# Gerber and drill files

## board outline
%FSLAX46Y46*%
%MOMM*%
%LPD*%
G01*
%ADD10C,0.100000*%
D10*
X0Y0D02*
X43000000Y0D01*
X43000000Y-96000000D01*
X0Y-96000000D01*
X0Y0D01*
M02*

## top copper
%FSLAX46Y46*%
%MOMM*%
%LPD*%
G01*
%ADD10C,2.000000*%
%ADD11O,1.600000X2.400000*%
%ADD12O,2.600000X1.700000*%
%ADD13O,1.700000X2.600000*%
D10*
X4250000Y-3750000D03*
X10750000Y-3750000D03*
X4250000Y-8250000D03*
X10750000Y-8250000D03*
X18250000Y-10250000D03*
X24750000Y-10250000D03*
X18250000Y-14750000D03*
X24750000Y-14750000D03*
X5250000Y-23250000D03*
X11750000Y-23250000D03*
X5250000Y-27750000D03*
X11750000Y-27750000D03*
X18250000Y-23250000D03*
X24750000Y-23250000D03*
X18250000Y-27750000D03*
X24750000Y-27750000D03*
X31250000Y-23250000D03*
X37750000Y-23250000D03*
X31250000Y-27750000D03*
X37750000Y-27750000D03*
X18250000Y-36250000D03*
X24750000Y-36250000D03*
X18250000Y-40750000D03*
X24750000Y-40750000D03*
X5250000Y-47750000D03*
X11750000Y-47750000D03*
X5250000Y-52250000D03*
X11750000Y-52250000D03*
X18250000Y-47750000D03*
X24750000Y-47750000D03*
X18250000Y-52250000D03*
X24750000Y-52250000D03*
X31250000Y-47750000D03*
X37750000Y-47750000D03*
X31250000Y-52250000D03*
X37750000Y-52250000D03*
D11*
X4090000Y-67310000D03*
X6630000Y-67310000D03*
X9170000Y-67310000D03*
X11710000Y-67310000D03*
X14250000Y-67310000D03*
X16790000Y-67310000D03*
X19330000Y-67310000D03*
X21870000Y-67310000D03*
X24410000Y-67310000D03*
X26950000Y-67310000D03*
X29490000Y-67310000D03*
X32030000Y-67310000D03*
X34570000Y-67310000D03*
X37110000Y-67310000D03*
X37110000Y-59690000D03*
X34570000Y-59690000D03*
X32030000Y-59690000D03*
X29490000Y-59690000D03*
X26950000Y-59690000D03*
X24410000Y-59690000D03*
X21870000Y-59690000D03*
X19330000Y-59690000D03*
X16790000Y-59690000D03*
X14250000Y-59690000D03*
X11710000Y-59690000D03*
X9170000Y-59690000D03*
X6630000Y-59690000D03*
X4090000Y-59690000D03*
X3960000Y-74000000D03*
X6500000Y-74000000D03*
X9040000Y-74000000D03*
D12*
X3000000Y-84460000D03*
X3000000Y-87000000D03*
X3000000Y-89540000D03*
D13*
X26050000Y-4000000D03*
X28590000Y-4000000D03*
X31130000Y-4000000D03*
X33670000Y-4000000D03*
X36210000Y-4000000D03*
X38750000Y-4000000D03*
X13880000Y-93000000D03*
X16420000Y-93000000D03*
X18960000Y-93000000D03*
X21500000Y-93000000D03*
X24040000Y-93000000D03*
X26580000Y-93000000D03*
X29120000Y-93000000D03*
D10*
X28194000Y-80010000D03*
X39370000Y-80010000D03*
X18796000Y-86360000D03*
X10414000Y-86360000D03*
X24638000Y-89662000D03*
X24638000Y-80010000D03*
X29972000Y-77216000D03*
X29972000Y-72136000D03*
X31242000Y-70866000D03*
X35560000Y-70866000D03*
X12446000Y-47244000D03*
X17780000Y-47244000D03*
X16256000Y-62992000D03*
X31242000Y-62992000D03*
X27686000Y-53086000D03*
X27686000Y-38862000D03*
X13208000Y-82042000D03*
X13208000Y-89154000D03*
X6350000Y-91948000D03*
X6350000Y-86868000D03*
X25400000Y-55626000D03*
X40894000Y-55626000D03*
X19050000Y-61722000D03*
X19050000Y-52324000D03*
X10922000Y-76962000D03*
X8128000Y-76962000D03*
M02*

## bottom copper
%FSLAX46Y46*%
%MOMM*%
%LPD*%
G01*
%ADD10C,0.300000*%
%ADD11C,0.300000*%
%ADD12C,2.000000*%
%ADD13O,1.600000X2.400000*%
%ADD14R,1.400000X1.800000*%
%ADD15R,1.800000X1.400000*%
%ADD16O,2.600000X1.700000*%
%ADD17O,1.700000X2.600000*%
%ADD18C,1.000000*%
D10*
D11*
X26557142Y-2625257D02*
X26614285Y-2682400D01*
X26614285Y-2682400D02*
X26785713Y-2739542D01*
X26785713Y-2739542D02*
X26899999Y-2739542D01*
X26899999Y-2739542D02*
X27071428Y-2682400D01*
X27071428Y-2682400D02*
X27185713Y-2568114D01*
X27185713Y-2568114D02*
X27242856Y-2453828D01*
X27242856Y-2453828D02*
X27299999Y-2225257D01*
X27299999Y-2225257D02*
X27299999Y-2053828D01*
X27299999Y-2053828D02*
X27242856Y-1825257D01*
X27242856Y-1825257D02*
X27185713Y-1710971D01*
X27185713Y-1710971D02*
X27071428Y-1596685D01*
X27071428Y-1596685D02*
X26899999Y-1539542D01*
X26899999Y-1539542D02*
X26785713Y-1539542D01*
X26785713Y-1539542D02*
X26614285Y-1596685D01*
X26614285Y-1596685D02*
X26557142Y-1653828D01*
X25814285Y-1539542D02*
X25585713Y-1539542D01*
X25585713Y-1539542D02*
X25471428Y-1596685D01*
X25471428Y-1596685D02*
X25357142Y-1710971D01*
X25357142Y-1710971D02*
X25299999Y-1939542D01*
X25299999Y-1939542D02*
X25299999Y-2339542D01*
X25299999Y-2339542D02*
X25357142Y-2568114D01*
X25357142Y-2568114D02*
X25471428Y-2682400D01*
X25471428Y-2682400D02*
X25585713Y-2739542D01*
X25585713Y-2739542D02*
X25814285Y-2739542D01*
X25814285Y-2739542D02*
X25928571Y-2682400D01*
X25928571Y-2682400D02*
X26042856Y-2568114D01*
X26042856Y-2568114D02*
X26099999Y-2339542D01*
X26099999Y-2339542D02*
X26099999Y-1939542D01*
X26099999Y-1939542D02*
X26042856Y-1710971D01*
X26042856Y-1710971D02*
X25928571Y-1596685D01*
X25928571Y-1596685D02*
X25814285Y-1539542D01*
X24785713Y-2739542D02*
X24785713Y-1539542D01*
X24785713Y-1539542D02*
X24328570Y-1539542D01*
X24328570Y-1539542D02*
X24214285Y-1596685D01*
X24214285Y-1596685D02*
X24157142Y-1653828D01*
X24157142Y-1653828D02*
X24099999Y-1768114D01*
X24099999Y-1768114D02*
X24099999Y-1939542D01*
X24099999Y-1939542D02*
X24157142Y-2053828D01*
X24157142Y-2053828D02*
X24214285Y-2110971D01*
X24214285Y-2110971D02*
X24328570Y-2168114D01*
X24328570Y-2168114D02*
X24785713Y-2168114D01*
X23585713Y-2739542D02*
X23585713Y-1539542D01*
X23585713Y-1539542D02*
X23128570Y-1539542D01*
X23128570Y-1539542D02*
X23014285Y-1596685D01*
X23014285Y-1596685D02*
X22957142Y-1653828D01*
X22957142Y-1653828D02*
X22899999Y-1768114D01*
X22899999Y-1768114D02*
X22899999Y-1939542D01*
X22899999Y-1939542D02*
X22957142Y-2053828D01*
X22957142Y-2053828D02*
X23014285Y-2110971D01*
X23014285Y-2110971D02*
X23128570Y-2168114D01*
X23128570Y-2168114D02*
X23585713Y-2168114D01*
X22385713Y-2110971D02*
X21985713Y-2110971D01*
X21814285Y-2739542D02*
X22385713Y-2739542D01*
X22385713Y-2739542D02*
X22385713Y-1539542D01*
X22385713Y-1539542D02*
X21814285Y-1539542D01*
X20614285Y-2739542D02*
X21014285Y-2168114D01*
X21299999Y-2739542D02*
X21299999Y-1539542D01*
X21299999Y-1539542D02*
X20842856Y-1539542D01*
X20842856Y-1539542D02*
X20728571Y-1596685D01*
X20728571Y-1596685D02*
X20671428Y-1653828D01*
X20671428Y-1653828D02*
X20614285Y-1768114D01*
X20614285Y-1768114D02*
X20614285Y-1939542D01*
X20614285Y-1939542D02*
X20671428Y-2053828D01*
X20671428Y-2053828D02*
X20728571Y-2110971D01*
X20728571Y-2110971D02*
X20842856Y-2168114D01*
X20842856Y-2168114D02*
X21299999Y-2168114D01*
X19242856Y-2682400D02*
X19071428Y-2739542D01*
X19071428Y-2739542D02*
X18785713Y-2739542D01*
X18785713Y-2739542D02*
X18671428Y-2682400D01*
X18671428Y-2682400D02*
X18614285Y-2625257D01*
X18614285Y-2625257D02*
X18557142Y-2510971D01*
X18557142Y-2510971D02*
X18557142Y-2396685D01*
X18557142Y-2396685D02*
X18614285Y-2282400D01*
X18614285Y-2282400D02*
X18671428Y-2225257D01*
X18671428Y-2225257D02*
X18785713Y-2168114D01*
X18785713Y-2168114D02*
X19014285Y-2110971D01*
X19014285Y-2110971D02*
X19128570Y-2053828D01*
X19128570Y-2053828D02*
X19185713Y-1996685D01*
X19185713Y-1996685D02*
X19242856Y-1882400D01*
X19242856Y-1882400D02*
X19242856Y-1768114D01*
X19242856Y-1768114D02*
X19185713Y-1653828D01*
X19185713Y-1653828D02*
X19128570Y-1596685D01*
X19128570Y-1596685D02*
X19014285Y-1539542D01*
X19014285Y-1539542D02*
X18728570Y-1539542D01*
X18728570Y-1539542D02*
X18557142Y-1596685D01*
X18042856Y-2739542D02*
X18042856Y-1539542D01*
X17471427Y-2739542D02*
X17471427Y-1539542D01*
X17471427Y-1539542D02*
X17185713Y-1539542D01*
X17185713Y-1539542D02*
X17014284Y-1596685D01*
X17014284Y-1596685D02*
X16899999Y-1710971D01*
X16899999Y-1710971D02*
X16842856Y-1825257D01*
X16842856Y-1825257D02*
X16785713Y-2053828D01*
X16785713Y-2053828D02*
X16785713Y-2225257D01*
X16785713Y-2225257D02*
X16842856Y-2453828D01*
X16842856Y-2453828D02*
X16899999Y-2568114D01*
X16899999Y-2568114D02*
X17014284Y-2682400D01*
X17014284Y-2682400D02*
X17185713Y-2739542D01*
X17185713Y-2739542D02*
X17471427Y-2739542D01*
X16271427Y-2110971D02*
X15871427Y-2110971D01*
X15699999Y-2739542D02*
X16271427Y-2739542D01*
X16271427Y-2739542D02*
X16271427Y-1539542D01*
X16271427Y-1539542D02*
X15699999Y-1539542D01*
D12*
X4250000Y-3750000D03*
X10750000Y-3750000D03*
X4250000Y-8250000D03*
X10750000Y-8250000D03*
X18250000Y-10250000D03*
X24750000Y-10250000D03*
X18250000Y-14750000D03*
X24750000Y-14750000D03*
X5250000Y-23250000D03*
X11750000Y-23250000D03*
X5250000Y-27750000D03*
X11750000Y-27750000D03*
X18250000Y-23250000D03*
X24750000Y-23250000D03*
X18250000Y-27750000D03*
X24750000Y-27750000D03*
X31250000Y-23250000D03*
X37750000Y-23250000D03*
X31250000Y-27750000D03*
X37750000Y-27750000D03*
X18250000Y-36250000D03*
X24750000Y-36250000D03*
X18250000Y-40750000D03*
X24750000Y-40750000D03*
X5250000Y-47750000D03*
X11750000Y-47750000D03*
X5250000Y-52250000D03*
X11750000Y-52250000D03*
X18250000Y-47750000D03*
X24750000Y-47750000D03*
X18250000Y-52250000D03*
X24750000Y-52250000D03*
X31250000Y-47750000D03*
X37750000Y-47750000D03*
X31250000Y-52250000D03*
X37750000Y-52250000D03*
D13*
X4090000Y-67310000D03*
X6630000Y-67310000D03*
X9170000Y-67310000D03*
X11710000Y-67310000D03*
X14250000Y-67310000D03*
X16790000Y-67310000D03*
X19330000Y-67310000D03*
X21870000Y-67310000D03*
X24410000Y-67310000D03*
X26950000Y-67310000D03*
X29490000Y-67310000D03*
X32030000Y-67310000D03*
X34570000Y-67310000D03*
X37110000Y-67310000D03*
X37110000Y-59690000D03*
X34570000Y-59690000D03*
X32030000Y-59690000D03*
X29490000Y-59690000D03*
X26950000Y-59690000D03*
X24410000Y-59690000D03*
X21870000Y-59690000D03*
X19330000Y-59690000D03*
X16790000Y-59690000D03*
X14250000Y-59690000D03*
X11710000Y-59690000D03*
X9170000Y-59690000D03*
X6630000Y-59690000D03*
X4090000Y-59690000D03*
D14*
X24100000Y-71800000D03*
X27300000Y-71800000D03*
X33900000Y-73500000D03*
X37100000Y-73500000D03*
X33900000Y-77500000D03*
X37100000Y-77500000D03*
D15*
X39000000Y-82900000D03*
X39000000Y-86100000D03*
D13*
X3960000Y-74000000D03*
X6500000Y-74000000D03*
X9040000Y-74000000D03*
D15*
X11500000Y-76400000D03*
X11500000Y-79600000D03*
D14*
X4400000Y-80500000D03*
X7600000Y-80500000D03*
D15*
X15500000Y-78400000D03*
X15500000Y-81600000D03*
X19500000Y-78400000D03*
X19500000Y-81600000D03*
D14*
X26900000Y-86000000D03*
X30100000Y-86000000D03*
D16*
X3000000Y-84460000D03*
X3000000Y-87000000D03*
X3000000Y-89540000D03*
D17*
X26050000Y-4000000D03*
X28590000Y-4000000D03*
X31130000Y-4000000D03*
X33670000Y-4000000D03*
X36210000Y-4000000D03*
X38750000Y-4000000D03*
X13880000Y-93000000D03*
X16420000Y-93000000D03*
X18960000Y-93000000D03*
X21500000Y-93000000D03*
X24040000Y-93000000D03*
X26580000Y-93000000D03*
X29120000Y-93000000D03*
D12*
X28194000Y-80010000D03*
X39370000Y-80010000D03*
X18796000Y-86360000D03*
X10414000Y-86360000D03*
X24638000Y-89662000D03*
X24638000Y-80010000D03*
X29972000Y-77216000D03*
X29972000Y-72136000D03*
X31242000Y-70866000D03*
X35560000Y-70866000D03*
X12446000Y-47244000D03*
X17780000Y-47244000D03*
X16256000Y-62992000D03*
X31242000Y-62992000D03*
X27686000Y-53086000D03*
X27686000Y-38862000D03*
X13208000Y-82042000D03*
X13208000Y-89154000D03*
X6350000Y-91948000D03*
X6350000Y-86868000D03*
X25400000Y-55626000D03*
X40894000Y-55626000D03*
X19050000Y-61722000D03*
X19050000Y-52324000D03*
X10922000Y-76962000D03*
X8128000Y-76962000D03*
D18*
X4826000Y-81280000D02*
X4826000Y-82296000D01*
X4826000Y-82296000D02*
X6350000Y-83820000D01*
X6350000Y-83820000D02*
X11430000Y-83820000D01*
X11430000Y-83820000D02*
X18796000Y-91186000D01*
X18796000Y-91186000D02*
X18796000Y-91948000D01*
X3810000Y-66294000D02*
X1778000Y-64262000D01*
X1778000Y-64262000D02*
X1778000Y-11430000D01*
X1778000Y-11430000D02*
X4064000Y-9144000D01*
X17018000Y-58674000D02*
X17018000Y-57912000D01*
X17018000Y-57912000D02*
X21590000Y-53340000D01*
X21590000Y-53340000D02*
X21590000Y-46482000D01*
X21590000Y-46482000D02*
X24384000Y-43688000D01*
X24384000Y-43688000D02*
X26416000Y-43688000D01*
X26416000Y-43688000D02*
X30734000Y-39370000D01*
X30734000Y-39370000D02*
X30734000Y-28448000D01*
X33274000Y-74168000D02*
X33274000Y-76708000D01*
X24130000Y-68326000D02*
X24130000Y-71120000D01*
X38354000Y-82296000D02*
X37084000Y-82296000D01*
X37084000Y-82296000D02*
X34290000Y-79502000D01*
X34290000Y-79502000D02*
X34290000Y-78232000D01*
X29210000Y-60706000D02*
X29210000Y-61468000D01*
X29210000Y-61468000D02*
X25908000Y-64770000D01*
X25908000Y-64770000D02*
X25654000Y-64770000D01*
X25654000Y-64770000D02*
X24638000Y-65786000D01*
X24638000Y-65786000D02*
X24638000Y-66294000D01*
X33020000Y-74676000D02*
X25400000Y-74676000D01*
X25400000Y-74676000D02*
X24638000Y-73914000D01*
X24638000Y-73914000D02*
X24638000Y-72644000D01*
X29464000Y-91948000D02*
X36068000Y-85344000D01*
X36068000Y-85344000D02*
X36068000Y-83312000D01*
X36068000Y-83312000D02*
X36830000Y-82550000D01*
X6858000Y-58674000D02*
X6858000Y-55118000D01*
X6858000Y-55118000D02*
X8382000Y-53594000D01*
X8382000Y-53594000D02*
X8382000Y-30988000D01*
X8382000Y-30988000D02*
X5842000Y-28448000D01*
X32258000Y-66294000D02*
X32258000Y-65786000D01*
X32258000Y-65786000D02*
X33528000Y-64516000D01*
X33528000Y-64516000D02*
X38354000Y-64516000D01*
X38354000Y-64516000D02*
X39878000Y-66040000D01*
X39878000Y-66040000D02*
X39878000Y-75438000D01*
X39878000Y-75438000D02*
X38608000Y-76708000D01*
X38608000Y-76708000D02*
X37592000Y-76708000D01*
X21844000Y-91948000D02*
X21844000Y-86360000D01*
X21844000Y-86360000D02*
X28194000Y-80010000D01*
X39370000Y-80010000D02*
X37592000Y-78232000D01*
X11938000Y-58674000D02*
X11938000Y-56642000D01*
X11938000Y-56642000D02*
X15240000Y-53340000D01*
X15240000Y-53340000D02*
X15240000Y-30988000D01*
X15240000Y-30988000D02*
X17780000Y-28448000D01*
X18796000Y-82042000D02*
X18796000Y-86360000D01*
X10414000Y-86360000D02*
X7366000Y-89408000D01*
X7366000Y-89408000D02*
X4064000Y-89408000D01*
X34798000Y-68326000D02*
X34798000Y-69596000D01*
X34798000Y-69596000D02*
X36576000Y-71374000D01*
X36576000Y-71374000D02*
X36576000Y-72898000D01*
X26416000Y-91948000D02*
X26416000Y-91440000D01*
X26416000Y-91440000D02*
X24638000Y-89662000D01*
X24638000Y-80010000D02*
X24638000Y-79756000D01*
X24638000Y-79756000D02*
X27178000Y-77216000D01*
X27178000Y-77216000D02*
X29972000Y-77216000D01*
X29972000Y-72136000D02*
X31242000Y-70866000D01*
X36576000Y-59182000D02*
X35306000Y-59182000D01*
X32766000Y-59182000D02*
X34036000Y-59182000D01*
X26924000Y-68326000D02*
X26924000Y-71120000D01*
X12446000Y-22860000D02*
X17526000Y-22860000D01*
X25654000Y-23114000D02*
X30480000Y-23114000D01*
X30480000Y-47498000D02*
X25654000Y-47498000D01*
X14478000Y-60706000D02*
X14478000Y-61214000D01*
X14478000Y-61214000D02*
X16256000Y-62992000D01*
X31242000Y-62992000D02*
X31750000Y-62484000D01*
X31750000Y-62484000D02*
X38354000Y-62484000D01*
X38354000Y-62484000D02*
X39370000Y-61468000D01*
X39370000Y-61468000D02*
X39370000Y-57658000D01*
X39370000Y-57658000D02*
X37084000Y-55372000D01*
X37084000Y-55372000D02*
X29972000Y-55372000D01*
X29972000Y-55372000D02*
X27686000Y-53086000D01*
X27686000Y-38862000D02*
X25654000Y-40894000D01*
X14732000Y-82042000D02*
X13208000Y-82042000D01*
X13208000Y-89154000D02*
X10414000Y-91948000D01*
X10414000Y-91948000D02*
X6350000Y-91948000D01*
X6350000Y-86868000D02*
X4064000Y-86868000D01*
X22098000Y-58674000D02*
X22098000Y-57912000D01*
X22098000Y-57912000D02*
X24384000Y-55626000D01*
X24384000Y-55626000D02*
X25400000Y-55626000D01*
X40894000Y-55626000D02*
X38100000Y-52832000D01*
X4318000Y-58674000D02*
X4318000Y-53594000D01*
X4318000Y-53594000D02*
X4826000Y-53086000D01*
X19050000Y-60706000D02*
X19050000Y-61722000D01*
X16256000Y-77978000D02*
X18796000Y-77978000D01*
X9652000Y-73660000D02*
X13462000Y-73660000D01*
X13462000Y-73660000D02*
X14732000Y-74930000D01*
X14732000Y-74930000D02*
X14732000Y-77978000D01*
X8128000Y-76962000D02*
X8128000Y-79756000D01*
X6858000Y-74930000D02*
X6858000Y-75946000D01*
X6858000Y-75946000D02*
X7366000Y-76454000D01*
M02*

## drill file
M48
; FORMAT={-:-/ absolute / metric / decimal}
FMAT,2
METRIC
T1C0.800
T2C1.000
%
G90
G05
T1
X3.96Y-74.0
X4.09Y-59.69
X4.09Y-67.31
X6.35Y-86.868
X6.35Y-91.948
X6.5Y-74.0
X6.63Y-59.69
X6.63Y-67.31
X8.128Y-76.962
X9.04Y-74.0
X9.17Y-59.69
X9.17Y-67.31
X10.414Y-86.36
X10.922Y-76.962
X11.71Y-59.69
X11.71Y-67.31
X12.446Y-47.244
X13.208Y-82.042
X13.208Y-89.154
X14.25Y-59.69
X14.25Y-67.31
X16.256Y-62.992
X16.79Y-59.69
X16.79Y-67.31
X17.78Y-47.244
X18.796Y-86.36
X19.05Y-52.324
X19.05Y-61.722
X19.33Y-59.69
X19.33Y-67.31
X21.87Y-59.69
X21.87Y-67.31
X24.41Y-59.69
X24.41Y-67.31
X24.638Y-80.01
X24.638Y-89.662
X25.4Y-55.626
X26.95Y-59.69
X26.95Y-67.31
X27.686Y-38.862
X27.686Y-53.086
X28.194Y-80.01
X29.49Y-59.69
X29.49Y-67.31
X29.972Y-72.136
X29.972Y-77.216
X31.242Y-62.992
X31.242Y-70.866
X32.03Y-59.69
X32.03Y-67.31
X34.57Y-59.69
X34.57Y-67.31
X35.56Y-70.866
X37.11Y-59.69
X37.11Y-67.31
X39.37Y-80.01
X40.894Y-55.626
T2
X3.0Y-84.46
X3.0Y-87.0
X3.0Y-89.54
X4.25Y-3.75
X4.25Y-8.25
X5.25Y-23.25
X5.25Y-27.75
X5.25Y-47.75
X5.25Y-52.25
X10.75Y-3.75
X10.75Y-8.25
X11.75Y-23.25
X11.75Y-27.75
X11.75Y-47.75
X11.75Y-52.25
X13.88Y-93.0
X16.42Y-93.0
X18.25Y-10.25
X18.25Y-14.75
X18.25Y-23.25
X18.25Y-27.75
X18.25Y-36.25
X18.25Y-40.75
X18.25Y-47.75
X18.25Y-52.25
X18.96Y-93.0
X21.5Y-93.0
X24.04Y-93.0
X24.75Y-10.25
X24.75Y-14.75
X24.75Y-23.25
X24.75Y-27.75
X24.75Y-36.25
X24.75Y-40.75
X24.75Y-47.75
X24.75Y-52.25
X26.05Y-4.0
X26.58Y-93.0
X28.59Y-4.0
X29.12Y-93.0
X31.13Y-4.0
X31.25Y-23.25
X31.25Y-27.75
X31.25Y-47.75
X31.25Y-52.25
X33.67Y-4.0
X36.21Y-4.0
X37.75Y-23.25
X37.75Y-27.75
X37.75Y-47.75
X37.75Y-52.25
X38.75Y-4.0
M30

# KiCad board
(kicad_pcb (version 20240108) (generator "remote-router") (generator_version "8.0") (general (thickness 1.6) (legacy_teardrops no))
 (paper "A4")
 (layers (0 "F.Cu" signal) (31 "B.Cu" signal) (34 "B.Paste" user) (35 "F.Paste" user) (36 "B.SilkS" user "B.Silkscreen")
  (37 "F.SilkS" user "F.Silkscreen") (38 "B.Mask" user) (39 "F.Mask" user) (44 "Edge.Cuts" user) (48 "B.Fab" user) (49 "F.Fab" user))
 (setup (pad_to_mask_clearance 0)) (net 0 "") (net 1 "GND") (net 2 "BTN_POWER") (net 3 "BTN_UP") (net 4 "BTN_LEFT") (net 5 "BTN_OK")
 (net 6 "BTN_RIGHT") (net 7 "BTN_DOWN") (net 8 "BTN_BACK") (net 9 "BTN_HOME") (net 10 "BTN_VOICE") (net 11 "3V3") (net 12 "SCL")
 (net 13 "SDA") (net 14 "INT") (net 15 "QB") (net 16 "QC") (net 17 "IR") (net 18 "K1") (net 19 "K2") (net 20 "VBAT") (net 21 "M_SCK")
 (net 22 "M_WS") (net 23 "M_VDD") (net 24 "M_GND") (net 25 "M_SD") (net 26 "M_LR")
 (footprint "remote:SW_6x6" (layer "F.Cu") (at 7.5000 6.0000)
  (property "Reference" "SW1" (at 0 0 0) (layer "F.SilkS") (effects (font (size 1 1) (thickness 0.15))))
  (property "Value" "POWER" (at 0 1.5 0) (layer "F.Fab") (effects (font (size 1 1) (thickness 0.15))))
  (pad "1" thru_hole circle (at -3.25 -2.25) (size 2.0 2.0) (drill 1.0) (layers "*.Cu" "*.Mask") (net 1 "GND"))
  (pad "2" thru_hole circle (at 3.25 -2.25) (size 2.0 2.0) (drill 1.0) (layers "*.Cu" "*.Mask") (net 1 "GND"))
  (pad "3" thru_hole circle (at -3.25 2.25) (size 2.0 2.0) (drill 1.0) (layers "*.Cu" "*.Mask") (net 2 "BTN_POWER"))
  (pad "4" thru_hole circle (at 3.25 2.25) (size 2.0 2.0) (drill 1.0) (layers "*.Cu" "*.Mask") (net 2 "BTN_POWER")))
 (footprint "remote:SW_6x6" (layer "F.Cu") (at 21.5000 12.5000)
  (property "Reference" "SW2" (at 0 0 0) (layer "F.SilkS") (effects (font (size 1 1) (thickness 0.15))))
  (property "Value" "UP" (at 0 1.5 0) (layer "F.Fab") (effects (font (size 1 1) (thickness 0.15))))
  (pad "1" thru_hole circle (at -3.25 -2.25) (size 2.0 2.0) (drill 1.0) (layers "*.Cu" "*.Mask") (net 1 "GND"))
  (pad "2" thru_hole circle (at 3.25 -2.25) (size 2.0 2.0) (drill 1.0) (layers "*.Cu" "*.Mask") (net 1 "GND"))
  (pad "3" thru_hole circle (at -3.25 2.25) (size 2.0 2.0) (drill 1.0) (layers "*.Cu" "*.Mask") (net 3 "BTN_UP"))
  (pad "4" thru_hole circle (at 3.25 2.25) (size 2.0 2.0) (drill 1.0) (layers "*.Cu" "*.Mask") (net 3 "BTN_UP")))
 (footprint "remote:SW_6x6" (layer "F.Cu") (at 8.5000 25.5000)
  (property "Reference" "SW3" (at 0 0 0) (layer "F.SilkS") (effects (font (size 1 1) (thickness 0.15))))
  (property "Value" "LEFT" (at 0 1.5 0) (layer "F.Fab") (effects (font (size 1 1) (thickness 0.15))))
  (pad "1" thru_hole circle (at -3.25 -2.25) (size 2.0 2.0) (drill 1.0) (layers "*.Cu" "*.Mask") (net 1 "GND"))
  (pad "2" thru_hole circle (at 3.25 -2.25) (size 2.0 2.0) (drill 1.0) (layers "*.Cu" "*.Mask") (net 1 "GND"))
  (pad "3" thru_hole circle (at -3.25 2.25) (size 2.0 2.0) (drill 1.0) (layers "*.Cu" "*.Mask") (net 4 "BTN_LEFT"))
  (pad "4" thru_hole circle (at 3.25 2.25) (size 2.0 2.0) (drill 1.0) (layers "*.Cu" "*.Mask") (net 4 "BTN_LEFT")))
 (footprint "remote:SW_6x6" (layer "F.Cu") (at 21.5000 25.5000)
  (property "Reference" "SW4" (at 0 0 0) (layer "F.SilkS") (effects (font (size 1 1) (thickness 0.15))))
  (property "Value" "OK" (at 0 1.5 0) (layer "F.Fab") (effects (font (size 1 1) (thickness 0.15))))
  (pad "1" thru_hole circle (at -3.25 -2.25) (size 2.0 2.0) (drill 1.0) (layers "*.Cu" "*.Mask") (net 1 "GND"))
  (pad "2" thru_hole circle (at 3.25 -2.25) (size 2.0 2.0) (drill 1.0) (layers "*.Cu" "*.Mask") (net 1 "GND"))
  (pad "3" thru_hole circle (at -3.25 2.25) (size 2.0 2.0) (drill 1.0) (layers "*.Cu" "*.Mask") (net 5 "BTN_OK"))
  (pad "4" thru_hole circle (at 3.25 2.25) (size 2.0 2.0) (drill 1.0) (layers "*.Cu" "*.Mask") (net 5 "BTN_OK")))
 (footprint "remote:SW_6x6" (layer "F.Cu") (at 34.5000 25.5000)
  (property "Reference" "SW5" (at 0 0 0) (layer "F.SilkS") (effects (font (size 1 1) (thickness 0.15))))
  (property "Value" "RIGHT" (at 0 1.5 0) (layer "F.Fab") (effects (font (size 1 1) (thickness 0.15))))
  (pad "1" thru_hole circle (at -3.25 -2.25) (size 2.0 2.0) (drill 1.0) (layers "*.Cu" "*.Mask") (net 1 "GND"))
  (pad "2" thru_hole circle (at 3.25 -2.25) (size 2.0 2.0) (drill 1.0) (layers "*.Cu" "*.Mask") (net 1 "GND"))
  (pad "3" thru_hole circle (at -3.25 2.25) (size 2.0 2.0) (drill 1.0) (layers "*.Cu" "*.Mask") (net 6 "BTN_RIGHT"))
  (pad "4" thru_hole circle (at 3.25 2.25) (size 2.0 2.0) (drill 1.0) (layers "*.Cu" "*.Mask") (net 6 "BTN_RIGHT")))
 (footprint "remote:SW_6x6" (layer "F.Cu") (at 21.5000 38.5000)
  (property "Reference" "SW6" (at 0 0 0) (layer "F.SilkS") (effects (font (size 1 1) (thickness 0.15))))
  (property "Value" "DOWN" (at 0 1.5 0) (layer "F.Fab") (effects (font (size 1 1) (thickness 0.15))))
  (pad "1" thru_hole circle (at -3.25 -2.25) (size 2.0 2.0) (drill 1.0) (layers "*.Cu" "*.Mask") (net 1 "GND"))
  (pad "2" thru_hole circle (at 3.25 -2.25) (size 2.0 2.0) (drill 1.0) (layers "*.Cu" "*.Mask") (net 1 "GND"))
  (pad "3" thru_hole circle (at -3.25 2.25) (size 2.0 2.0) (drill 1.0) (layers "*.Cu" "*.Mask") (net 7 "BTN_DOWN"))
  (pad "4" thru_hole circle (at 3.25 2.25) (size 2.0 2.0) (drill 1.0) (layers "*.Cu" "*.Mask") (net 7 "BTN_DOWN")))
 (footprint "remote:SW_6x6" (layer "F.Cu") (at 8.5000 50.0000)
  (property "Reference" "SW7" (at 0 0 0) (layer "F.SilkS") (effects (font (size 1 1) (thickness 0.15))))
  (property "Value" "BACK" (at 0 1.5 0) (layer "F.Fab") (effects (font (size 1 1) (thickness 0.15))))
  (pad "1" thru_hole circle (at -3.25 -2.25) (size 2.0 2.0) (drill 1.0) (layers "*.Cu" "*.Mask") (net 1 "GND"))
  (pad "2" thru_hole circle (at 3.25 -2.25) (size 2.0 2.0) (drill 1.0) (layers "*.Cu" "*.Mask") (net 1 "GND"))
  (pad "3" thru_hole circle (at -3.25 2.25) (size 2.0 2.0) (drill 1.0) (layers "*.Cu" "*.Mask") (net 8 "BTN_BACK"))
  (pad "4" thru_hole circle (at 3.25 2.25) (size 2.0 2.0) (drill 1.0) (layers "*.Cu" "*.Mask") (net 8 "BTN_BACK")))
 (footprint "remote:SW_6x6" (layer "F.Cu") (at 21.5000 50.0000)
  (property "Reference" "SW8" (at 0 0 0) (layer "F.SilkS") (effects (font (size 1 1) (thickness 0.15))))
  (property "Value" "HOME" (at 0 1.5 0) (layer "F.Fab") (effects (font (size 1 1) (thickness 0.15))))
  (pad "1" thru_hole circle (at -3.25 -2.25) (size 2.0 2.0) (drill 1.0) (layers "*.Cu" "*.Mask") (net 1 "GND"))
  (pad "2" thru_hole circle (at 3.25 -2.25) (size 2.0 2.0) (drill 1.0) (layers "*.Cu" "*.Mask") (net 1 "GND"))
  (pad "3" thru_hole circle (at -3.25 2.25) (size 2.0 2.0) (drill 1.0) (layers "*.Cu" "*.Mask") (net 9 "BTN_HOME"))
  (pad "4" thru_hole circle (at 3.25 2.25) (size 2.0 2.0) (drill 1.0) (layers "*.Cu" "*.Mask") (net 9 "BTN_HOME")))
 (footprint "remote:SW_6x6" (layer "F.Cu") (at 34.5000 50.0000)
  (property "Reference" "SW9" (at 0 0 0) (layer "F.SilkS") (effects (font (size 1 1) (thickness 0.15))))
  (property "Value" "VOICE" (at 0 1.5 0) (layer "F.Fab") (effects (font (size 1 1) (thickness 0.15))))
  (pad "1" thru_hole circle (at -3.25 -2.25) (size 2.0 2.0) (drill 1.0) (layers "*.Cu" "*.Mask") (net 1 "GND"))
  (pad "2" thru_hole circle (at 3.25 -2.25) (size 2.0 2.0) (drill 1.0) (layers "*.Cu" "*.Mask") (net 1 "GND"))
  (pad "3" thru_hole circle (at -3.25 2.25) (size 2.0 2.0) (drill 1.0) (layers "*.Cu" "*.Mask") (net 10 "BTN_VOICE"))
  (pad "4" thru_hole circle (at 3.25 2.25) (size 2.0 2.0) (drill 1.0) (layers "*.Cu" "*.Mask") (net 10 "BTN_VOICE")))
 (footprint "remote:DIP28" (layer "F.Cu") (at 20.6000 63.5000)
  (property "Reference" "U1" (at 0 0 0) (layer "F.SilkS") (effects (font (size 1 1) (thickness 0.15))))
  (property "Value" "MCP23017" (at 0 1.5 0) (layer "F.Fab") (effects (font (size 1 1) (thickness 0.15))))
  (pad "1" thru_hole oval (at -16.51 3.81) (size 1.6 2.4) (drill 0.8) (layers "*.Cu" "*.Mask") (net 2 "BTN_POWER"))
  (pad "2" thru_hole oval (at -13.97 3.81) (size 1.6 2.4) (drill 0.8) (layers "*.Cu" "*.Mask"))
  (pad "3" thru_hole oval (at -11.43 3.81) (size 1.6 2.4) (drill 0.8) (layers "*.Cu" "*.Mask"))
  (pad "4" thru_hole oval (at -8.89 3.81) (size 1.6 2.4) (drill 0.8) (layers "*.Cu" "*.Mask"))
  (pad "5" thru_hole oval (at -6.35 3.81) (size 1.6 2.4) (drill 0.8) (layers "*.Cu" "*.Mask"))
  (pad "6" thru_hole oval (at -3.81 3.81) (size 1.6 2.4) (drill 0.8) (layers "*.Cu" "*.Mask"))
  (pad "7" thru_hole oval (at -1.27 3.81) (size 1.6 2.4) (drill 0.8) (layers "*.Cu" "*.Mask"))
  (pad "8" thru_hole oval (at 1.27 3.81) (size 1.6 2.4) (drill 0.8) (layers "*.Cu" "*.Mask"))
  (pad "9" thru_hole oval (at 3.81 3.81) (size 1.6 2.4) (drill 0.8) (layers "*.Cu" "*.Mask") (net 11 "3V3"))
  (pad "10" thru_hole oval (at 6.35 3.81) (size 1.6 2.4) (drill 0.8) (layers "*.Cu" "*.Mask") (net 1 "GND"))
  (pad "11" thru_hole oval (at 8.89 3.81) (size 1.6 2.4) (drill 0.8) (layers "*.Cu" "*.Mask"))
  (pad "12" thru_hole oval (at 11.43 3.81) (size 1.6 2.4) (drill 0.8) (layers "*.Cu" "*.Mask") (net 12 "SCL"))
  (pad "13" thru_hole oval (at 13.97 3.81) (size 1.6 2.4) (drill 0.8) (layers "*.Cu" "*.Mask") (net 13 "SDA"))
  (pad "14" thru_hole oval (at 16.51 3.81) (size 1.6 2.4) (drill 0.8) (layers "*.Cu" "*.Mask"))
  (pad "15" thru_hole oval (at 16.51 -3.81) (size 1.6 2.4) (drill 0.8) (layers "*.Cu" "*.Mask") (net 1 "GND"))
  (pad "16" thru_hole oval (at 13.97 -3.81) (size 1.6 2.4) (drill 0.8) (layers "*.Cu" "*.Mask") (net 1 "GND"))
  (pad "17" thru_hole oval (at 11.43 -3.81) (size 1.6 2.4) (drill 0.8) (layers "*.Cu" "*.Mask") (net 1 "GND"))
  (pad "18" thru_hole oval (at 8.89 -3.81) (size 1.6 2.4) (drill 0.8) (layers "*.Cu" "*.Mask") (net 11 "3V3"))
  (pad "19" thru_hole oval (at 6.35 -3.81) (size 1.6 2.4) (drill 0.8) (layers "*.Cu" "*.Mask"))
  (pad "20" thru_hole oval (at 3.81 -3.81) (size 1.6 2.4) (drill 0.8) (layers "*.Cu" "*.Mask") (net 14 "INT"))
  (pad "21" thru_hole oval (at 1.27 -3.81) (size 1.6 2.4) (drill 0.8) (layers "*.Cu" "*.Mask") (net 10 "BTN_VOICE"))
  (pad "22" thru_hole oval (at -1.27 -3.81) (size 1.6 2.4) (drill 0.8) (layers "*.Cu" "*.Mask") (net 9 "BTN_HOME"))
  (pad "23" thru_hole oval (at -3.81 -3.81) (size 1.6 2.4) (drill 0.8) (layers "*.Cu" "*.Mask") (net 6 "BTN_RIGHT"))
  (pad "24" thru_hole oval (at -6.35 -3.81) (size 1.6 2.4) (drill 0.8) (layers "*.Cu" "*.Mask") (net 7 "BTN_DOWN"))
  (pad "25" thru_hole oval (at -8.89 -3.81) (size 1.6 2.4) (drill 0.8) (layers "*.Cu" "*.Mask") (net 5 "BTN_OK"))
  (pad "26" thru_hole oval (at -11.43 -3.81) (size 1.6 2.4) (drill 0.8) (layers "*.Cu" "*.Mask") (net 3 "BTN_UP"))
  (pad "27" thru_hole oval (at -13.97 -3.81) (size 1.6 2.4) (drill 0.8) (layers "*.Cu" "*.Mask") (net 4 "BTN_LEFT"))
  (pad "28" thru_hole oval (at -16.51 -3.81) (size 1.6 2.4) (drill 0.8) (layers "*.Cu" "*.Mask") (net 8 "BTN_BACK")))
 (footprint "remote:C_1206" (layer "F.Cu") (at 25.7000 71.8000)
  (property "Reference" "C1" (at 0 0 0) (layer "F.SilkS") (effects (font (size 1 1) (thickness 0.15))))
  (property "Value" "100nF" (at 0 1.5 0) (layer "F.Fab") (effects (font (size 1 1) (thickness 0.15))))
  (pad "1" smd rect (at -1.6 0.0) (size 1.4 1.8) (layers "B.Cu" "B.Mask") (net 11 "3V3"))
  (pad "2" smd rect (at 1.6 0.0) (size 1.4 1.8) (layers "B.Cu" "B.Mask") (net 1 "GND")))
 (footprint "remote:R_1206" (layer "F.Cu") (at 35.5000 73.5000)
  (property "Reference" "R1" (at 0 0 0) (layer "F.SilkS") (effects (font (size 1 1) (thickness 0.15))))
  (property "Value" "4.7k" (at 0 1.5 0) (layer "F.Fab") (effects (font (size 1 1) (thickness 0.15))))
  (pad "1" smd rect (at -1.6 0.0) (size 1.4 1.8) (layers "B.Cu" "B.Mask") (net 11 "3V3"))
  (pad "2" smd rect (at 1.6 0.0) (size 1.4 1.8) (layers "B.Cu" "B.Mask") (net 13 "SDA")))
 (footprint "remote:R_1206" (layer "F.Cu") (at 35.5000 77.5000)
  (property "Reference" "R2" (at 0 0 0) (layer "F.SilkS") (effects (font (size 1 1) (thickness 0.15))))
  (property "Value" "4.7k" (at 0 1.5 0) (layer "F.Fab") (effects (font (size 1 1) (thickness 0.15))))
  (pad "1" smd rect (at -1.6 0.0) (size 1.4 1.8) (layers "B.Cu" "B.Mask") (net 11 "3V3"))
  (pad "2" smd rect (at 1.6 0.0) (size 1.4 1.8) (layers "B.Cu" "B.Mask") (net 12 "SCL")))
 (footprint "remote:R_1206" (layer "F.Cu") (at 39.0000 84.5000)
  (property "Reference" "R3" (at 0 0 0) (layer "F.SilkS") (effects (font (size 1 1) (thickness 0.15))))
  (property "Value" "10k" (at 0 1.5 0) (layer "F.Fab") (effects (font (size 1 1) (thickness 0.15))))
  (pad "1" smd rect (at 0.0 -1.6) (size 1.8 1.4) (layers "B.Cu" "B.Mask") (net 11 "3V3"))
  (pad "2" smd rect (at 0.0 1.6) (size 1.8 1.4) (layers "B.Cu" "B.Mask") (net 14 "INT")))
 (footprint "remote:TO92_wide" (layer "F.Cu") (at 6.5000 74.0000)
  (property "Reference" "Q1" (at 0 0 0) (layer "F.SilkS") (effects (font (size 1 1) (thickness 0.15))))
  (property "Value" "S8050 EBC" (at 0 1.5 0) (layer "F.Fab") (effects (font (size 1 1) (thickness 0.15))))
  (pad "E" thru_hole oval (at -2.54 0.0) (size 1.6 2.4) (drill 0.8) (layers "*.Cu" "*.Mask") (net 1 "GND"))
  (pad "B" thru_hole oval (at 0.0 0.0) (size 1.6 2.4) (drill 0.8) (layers "*.Cu" "*.Mask") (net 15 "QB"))
  (pad "C" thru_hole oval (at 2.54 0.0) (size 1.6 2.4) (drill 0.8) (layers "*.Cu" "*.Mask") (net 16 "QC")))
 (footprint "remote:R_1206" (layer "F.Cu") (at 11.5000 78.0000)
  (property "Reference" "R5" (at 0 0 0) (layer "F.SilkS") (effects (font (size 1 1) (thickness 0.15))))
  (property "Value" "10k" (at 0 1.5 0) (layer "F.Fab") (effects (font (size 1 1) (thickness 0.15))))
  (pad "1" smd rect (at 0.0 -1.6) (size 1.8 1.4) (layers "B.Cu" "B.Mask") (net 15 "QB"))
  (pad "2" smd rect (at 0.0 1.6) (size 1.8 1.4) (layers "B.Cu" "B.Mask") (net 1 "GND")))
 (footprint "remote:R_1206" (layer "F.Cu") (at 6.0000 80.5000)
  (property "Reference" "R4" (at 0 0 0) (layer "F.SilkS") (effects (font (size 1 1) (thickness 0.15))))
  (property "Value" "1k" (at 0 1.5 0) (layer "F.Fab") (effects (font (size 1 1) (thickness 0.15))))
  (pad "1" smd rect (at -1.6 0.0) (size 1.4 1.8) (layers "B.Cu" "B.Mask") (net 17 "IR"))
  (pad "2" smd rect (at 1.6 0.0) (size 1.4 1.8) (layers "B.Cu" "B.Mask") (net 15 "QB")))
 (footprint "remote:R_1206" (layer "F.Cu") (at 15.5000 80.0000)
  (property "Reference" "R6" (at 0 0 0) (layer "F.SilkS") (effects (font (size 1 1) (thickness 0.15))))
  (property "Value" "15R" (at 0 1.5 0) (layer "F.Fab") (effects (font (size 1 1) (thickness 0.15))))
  (pad "1" smd rect (at 0.0 -1.6) (size 1.8 1.4) (layers "B.Cu" "B.Mask") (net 16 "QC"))
  (pad "2" smd rect (at 0.0 1.6) (size 1.8 1.4) (layers "B.Cu" "B.Mask") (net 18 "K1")))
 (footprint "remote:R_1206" (layer "F.Cu") (at 19.5000 80.0000)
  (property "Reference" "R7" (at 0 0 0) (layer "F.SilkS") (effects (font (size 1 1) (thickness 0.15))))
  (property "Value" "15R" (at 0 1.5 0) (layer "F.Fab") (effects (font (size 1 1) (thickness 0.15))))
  (pad "1" smd rect (at 0.0 -1.6) (size 1.8 1.4) (layers "B.Cu" "B.Mask") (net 16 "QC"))
  (pad "2" smd rect (at 0.0 1.6) (size 1.8 1.4) (layers "B.Cu" "B.Mask") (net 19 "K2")))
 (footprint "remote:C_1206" (layer "F.Cu") (at 28.5000 86.0000)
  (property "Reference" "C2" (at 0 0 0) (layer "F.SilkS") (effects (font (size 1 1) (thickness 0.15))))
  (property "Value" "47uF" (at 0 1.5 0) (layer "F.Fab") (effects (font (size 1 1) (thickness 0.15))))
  (pad "1" smd rect (at -1.6 0.0) (size 1.4 1.8) (layers "B.Cu" "B.Mask") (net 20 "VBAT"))
  (pad "2" smd rect (at 1.6 0.0) (size 1.4 1.8) (layers "B.Cu" "B.Mask") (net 1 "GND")))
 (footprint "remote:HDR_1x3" (layer "F.Cu") (at 3.0000 87.0000)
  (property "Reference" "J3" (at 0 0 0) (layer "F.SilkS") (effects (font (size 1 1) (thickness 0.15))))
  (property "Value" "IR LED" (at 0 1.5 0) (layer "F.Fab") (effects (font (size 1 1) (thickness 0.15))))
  (pad "1" thru_hole oval (at 0.0 -2.54) (size 2.6 1.7) (drill 1.0) (layers "*.Cu" "*.Mask") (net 20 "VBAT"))
  (pad "2" thru_hole oval (at 0.0 0.0) (size 2.6 1.7) (drill 1.0) (layers "*.Cu" "*.Mask") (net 18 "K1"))
  (pad "3" thru_hole oval (at 0.0 2.54) (size 2.6 1.7) (drill 1.0) (layers "*.Cu" "*.Mask") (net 19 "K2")))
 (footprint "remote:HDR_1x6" (layer "F.Cu") (at 32.4000 4.0000)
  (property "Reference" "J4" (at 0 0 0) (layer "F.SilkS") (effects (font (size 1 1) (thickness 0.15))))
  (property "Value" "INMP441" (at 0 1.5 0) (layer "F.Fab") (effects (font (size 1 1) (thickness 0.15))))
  (pad "1" thru_hole oval (at -6.35 0.0) (size 1.7 2.6) (drill 1.0) (layers "*.Cu" "*.Mask") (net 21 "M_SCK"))
  (pad "2" thru_hole oval (at -3.81 0.0) (size 1.7 2.6) (drill 1.0) (layers "*.Cu" "*.Mask") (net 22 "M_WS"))
  (pad "3" thru_hole oval (at -1.27 0.0) (size 1.7 2.6) (drill 1.0) (layers "*.Cu" "*.Mask") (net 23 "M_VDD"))
  (pad "4" thru_hole oval (at 1.27 0.0) (size 1.7 2.6) (drill 1.0) (layers "*.Cu" "*.Mask") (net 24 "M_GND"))
  (pad "5" thru_hole oval (at 3.81 0.0) (size 1.7 2.6) (drill 1.0) (layers "*.Cu" "*.Mask") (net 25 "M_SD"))
  (pad "6" thru_hole oval (at 6.35 0.0) (size 1.7 2.6) (drill 1.0) (layers "*.Cu" "*.Mask") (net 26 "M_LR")))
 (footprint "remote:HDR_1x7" (layer "F.Cu") (at 21.5000 93.0000)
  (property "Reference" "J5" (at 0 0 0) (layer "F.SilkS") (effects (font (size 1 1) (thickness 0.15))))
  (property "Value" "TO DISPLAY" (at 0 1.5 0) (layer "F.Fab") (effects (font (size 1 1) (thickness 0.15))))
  (pad "1" thru_hole oval (at -7.62 0.0) (size 1.7 2.6) (drill 1.0) (layers "*.Cu" "*.Mask") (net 20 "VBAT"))
  (pad "2" thru_hole oval (at -5.08 0.0) (size 1.7 2.6) (drill 1.0) (layers "*.Cu" "*.Mask") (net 14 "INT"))
  (pad "3" thru_hole oval (at -2.54 0.0) (size 1.7 2.6) (drill 1.0) (layers "*.Cu" "*.Mask") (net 17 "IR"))
  (pad "4" thru_hole oval (at 0.0 0.0) (size 1.7 2.6) (drill 1.0) (layers "*.Cu" "*.Mask") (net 12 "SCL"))
  (pad "5" thru_hole oval (at 2.54 0.0) (size 1.7 2.6) (drill 1.0) (layers "*.Cu" "*.Mask") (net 1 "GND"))
  (pad "6" thru_hole oval (at 5.08 0.0) (size 1.7 2.6) (drill 1.0) (layers "*.Cu" "*.Mask") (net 13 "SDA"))
  (pad "7" thru_hole oval (at 7.62 0.0) (size 1.7 2.6) (drill 1.0) (layers "*.Cu" "*.Mask") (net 11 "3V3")))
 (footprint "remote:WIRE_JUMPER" (layer "F.Cu") (at 33.7820 80.0100)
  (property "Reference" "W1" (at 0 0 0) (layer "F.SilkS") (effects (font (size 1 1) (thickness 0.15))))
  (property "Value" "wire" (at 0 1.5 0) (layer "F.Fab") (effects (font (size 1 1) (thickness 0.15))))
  (pad "1" thru_hole circle (at -5.588 0.0) (size 2.0 2.0) (drill 0.8) (layers "*.Cu" "*.Mask") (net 12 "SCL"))
  (pad "2" thru_hole circle (at 5.588 0.0) (size 2.0 2.0) (drill 0.8) (layers "*.Cu" "*.Mask") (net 12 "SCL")))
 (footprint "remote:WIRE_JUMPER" (layer "F.Cu") (at 14.6050 86.3600)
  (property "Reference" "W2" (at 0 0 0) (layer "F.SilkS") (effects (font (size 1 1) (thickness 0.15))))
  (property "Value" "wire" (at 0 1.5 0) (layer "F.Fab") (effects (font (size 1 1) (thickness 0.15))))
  (pad "1" thru_hole circle (at 4.191 0.0) (size 2.0 2.0) (drill 0.8) (layers "*.Cu" "*.Mask") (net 19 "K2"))
  (pad "2" thru_hole circle (at -4.191 0.0) (size 2.0 2.0) (drill 0.8) (layers "*.Cu" "*.Mask") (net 19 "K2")))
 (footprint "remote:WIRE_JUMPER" (layer "F.Cu") (at 24.6380 84.8360)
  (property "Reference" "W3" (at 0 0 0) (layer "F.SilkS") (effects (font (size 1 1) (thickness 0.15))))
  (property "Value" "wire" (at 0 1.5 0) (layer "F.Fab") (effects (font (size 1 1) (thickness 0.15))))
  (pad "1" thru_hole circle (at 0.0 4.826) (size 2.0 2.0) (drill 0.8) (layers "*.Cu" "*.Mask") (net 13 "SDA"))
  (pad "2" thru_hole circle (at 0.0 -4.826) (size 2.0 2.0) (drill 0.8) (layers "*.Cu" "*.Mask") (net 13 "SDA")))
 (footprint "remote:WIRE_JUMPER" (layer "F.Cu") (at 29.9720 74.6760)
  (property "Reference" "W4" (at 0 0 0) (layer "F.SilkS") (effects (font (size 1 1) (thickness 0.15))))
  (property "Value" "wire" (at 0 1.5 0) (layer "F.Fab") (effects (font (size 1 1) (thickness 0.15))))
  (pad "1" thru_hole circle (at 0.0 2.54) (size 2.0 2.0) (drill 0.8) (layers "*.Cu" "*.Mask") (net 13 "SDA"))
  (pad "2" thru_hole circle (at 0.0 -2.54) (size 2.0 2.0) (drill 0.8) (layers "*.Cu" "*.Mask") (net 13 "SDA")))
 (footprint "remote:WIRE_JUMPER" (layer "F.Cu") (at 33.4010 70.8660)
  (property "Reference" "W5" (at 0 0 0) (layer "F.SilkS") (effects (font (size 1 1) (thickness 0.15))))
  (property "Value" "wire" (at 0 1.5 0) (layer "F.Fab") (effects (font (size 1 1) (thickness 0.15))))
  (pad "1" thru_hole circle (at -2.159 0.0) (size 2.0 2.0) (drill 0.8) (layers "*.Cu" "*.Mask") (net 13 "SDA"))
  (pad "2" thru_hole circle (at 2.159 0.0) (size 2.0 2.0) (drill 0.8) (layers "*.Cu" "*.Mask") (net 13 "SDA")))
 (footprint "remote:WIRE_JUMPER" (layer "F.Cu") (at 15.1130 47.2440)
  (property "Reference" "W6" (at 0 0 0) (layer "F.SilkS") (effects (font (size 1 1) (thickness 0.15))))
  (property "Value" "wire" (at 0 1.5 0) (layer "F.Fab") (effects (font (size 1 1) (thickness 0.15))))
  (pad "1" thru_hole circle (at -2.667 0.0) (size 2.0 2.0) (drill 0.8) (layers "*.Cu" "*.Mask") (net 1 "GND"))
  (pad "2" thru_hole circle (at 2.667 0.0) (size 2.0 2.0) (drill 0.8) (layers "*.Cu" "*.Mask") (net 1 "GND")))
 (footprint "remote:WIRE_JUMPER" (layer "F.Cu") (at 23.7490 62.9920)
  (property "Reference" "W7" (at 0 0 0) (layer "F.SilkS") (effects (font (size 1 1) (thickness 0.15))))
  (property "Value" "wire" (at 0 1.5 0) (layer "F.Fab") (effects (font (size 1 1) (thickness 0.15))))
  (pad "1" thru_hole circle (at -7.493 0.0) (size 2.0 2.0) (drill 0.8) (layers "*.Cu" "*.Mask") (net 7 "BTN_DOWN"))
  (pad "2" thru_hole circle (at 7.493 0.0) (size 2.0 2.0) (drill 0.8) (layers "*.Cu" "*.Mask") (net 7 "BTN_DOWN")))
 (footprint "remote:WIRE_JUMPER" (layer "F.Cu") (at 27.6860 45.9740)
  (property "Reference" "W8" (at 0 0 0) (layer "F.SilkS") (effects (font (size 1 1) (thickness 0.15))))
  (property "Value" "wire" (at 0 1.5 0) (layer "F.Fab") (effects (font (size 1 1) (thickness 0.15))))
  (pad "1" thru_hole circle (at 0.0 7.112) (size 2.0 2.0) (drill 0.8) (layers "*.Cu" "*.Mask") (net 7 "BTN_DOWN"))
  (pad "2" thru_hole circle (at 0.0 -7.112) (size 2.0 2.0) (drill 0.8) (layers "*.Cu" "*.Mask") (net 7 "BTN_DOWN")))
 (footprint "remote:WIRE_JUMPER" (layer "F.Cu") (at 13.2080 85.5980)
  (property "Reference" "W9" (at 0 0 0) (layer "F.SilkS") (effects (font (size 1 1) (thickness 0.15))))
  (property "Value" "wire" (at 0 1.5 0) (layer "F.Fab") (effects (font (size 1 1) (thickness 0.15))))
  (pad "1" thru_hole circle (at 0.0 -3.556) (size 2.0 2.0) (drill 0.8) (layers "*.Cu" "*.Mask") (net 18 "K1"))
  (pad "2" thru_hole circle (at 0.0 3.556) (size 2.0 2.0) (drill 0.8) (layers "*.Cu" "*.Mask") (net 18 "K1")))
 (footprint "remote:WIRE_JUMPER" (layer "F.Cu") (at 6.3500 89.4080)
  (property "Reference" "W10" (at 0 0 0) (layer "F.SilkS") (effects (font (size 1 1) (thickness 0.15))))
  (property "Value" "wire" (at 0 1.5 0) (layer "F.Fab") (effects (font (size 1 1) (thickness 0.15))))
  (pad "1" thru_hole circle (at 0.0 2.54) (size 2.0 2.0) (drill 0.8) (layers "*.Cu" "*.Mask") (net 18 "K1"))
  (pad "2" thru_hole circle (at 0.0 -2.54) (size 2.0 2.0) (drill 0.8) (layers "*.Cu" "*.Mask") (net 18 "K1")))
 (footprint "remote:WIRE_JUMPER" (layer "F.Cu") (at 33.1470 55.6260)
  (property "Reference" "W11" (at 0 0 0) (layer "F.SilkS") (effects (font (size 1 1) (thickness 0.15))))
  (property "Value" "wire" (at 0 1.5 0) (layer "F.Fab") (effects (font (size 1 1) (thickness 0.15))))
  (pad "1" thru_hole circle (at -7.747 0.0) (size 2.0 2.0) (drill 0.8) (layers "*.Cu" "*.Mask") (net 10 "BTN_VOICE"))
  (pad "2" thru_hole circle (at 7.747 0.0) (size 2.0 2.0) (drill 0.8) (layers "*.Cu" "*.Mask") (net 10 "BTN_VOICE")))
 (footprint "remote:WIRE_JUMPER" (layer "F.Cu") (at 19.0500 57.0230)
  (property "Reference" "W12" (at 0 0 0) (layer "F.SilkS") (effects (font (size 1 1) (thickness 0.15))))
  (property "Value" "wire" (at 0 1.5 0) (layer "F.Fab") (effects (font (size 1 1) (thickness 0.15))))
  (pad "1" thru_hole circle (at 0.0 4.699) (size 2.0 2.0) (drill 0.8) (layers "*.Cu" "*.Mask") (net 9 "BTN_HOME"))
  (pad "2" thru_hole circle (at 0.0 -4.699) (size 2.0 2.0) (drill 0.8) (layers "*.Cu" "*.Mask") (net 9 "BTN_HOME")))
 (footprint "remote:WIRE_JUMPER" (layer "F.Cu") (at 9.5250 76.9620)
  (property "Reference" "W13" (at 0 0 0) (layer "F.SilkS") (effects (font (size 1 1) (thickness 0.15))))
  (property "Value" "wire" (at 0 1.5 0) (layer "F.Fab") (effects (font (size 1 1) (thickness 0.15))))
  (pad "1" thru_hole circle (at 1.397 0.0) (size 2.0 2.0) (drill 0.8) (layers "*.Cu" "*.Mask") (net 15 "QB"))
  (pad "2" thru_hole circle (at -1.397 0.0) (size 2.0 2.0) (drill 0.8) (layers "*.Cu" "*.Mask") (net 15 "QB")))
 (segment (start 4.8260 81.2800) (end 4.8260 82.2960) (width 1.0) (layer "B.Cu") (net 17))
 (segment (start 4.8260 82.2960) (end 6.3500 83.8200) (width 1.0) (layer "B.Cu") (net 17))
 (segment (start 6.3500 83.8200) (end 11.4300 83.8200) (width 1.0) (layer "B.Cu") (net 17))
 (segment (start 11.4300 83.8200) (end 18.7960 91.1860) (width 1.0) (layer "B.Cu") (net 17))
 (segment (start 18.7960 91.1860) (end 18.7960 91.9480) (width 1.0) (layer "B.Cu") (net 17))
 (segment (start 3.8100 66.2940) (end 1.7780 64.2620) (width 1.0) (layer "B.Cu") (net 2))
 (segment (start 1.7780 64.2620) (end 1.7780 11.4300) (width 1.0) (layer "B.Cu") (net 2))
 (segment (start 1.7780 11.4300) (end 4.0640 9.1440) (width 1.0) (layer "B.Cu") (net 2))
 (segment (start 17.0180 58.6740) (end 17.0180 57.9120) (width 1.0) (layer "B.Cu") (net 6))
 (segment (start 17.0180 57.9120) (end 21.5900 53.3400) (width 1.0) (layer "B.Cu") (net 6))
 (segment (start 21.5900 53.3400) (end 21.5900 46.4820) (width 1.0) (layer "B.Cu") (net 6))
 (segment (start 21.5900 46.4820) (end 24.3840 43.6880) (width 1.0) (layer "B.Cu") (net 6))
 (segment (start 24.3840 43.6880) (end 26.4160 43.6880) (width 1.0) (layer "B.Cu") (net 6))
 (segment (start 26.4160 43.6880) (end 30.7340 39.3700) (width 1.0) (layer "B.Cu") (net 6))
 (segment (start 30.7340 39.3700) (end 30.7340 28.4480) (width 1.0) (layer "B.Cu") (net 6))
 (segment (start 33.2740 74.1680) (end 33.2740 76.7080) (width 1.0) (layer "B.Cu") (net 11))
 (segment (start 24.1300 68.3260) (end 24.1300 71.1200) (width 1.0) (layer "B.Cu") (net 11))
 (segment (start 38.3540 82.2960) (end 37.0840 82.2960) (width 1.0) (layer "B.Cu") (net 11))
 (segment (start 37.0840 82.2960) (end 34.2900 79.5020) (width 1.0) (layer "B.Cu") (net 11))
 (segment (start 34.2900 79.5020) (end 34.2900 78.2320) (width 1.0) (layer "B.Cu") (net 11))
 (segment (start 29.2100 60.7060) (end 29.2100 61.4680) (width 1.0) (layer "B.Cu") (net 11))
 (segment (start 29.2100 61.4680) (end 25.9080 64.7700) (width 1.0) (layer "B.Cu") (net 11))
 (segment (start 25.9080 64.7700) (end 25.6540 64.7700) (width 1.0) (layer "B.Cu") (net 11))
 (segment (start 25.6540 64.7700) (end 24.6380 65.7860) (width 1.0) (layer "B.Cu") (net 11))
 (segment (start 24.6380 65.7860) (end 24.6380 66.2940) (width 1.0) (layer "B.Cu") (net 11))
 (segment (start 33.0200 74.6760) (end 25.4000 74.6760) (width 1.0) (layer "B.Cu") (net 11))
 (segment (start 25.4000 74.6760) (end 24.6380 73.9140) (width 1.0) (layer "B.Cu") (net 11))
 (segment (start 24.6380 73.9140) (end 24.6380 72.6440) (width 1.0) (layer "B.Cu") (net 11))
 (segment (start 29.4640 91.9480) (end 36.0680 85.3440) (width 1.0) (layer "B.Cu") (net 11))
 (segment (start 36.0680 85.3440) (end 36.0680 83.3120) (width 1.0) (layer "B.Cu") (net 11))
 (segment (start 36.0680 83.3120) (end 36.8300 82.5500) (width 1.0) (layer "B.Cu") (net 11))
 (segment (start 6.8580 58.6740) (end 6.8580 55.1180) (width 1.0) (layer "B.Cu") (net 4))
 (segment (start 6.8580 55.1180) (end 8.3820 53.5940) (width 1.0) (layer "B.Cu") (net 4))
 (segment (start 8.3820 53.5940) (end 8.3820 30.9880) (width 1.0) (layer "B.Cu") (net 4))
 (segment (start 8.3820 30.9880) (end 5.8420 28.4480) (width 1.0) (layer "B.Cu") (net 4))
 (segment (start 32.2580 66.2940) (end 32.2580 65.7860) (width 1.0) (layer "B.Cu") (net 12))
 (segment (start 32.2580 65.7860) (end 33.5280 64.5160) (width 1.0) (layer "B.Cu") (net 12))
 (segment (start 33.5280 64.5160) (end 38.3540 64.5160) (width 1.0) (layer "B.Cu") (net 12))
 (segment (start 38.3540 64.5160) (end 39.8780 66.0400) (width 1.0) (layer "B.Cu") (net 12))
 (segment (start 39.8780 66.0400) (end 39.8780 75.4380) (width 1.0) (layer "B.Cu") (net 12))
 (segment (start 39.8780 75.4380) (end 38.6080 76.7080) (width 1.0) (layer "B.Cu") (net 12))
 (segment (start 38.6080 76.7080) (end 37.5920 76.7080) (width 1.0) (layer "B.Cu") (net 12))
 (segment (start 21.8440 91.9480) (end 21.8440 86.3600) (width 1.0) (layer "B.Cu") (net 12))
 (segment (start 21.8440 86.3600) (end 28.1940 80.0100) (width 1.0) (layer "B.Cu") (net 12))
 (segment (start 39.3700 80.0100) (end 37.5920 78.2320) (width 1.0) (layer "B.Cu") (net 12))
 (segment (start 11.9380 58.6740) (end 11.9380 56.6420) (width 1.0) (layer "B.Cu") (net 5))
 (segment (start 11.9380 56.6420) (end 15.2400 53.3400) (width 1.0) (layer "B.Cu") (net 5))
 (segment (start 15.2400 53.3400) (end 15.2400 30.9880) (width 1.0) (layer "B.Cu") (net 5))
 (segment (start 15.2400 30.9880) (end 17.7800 28.4480) (width 1.0) (layer "B.Cu") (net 5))
 (segment (start 18.7960 82.0420) (end 18.7960 86.3600) (width 1.0) (layer "B.Cu") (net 19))
 (segment (start 10.4140 86.3600) (end 7.3660 89.4080) (width 1.0) (layer "B.Cu") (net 19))
 (segment (start 7.3660 89.4080) (end 4.0640 89.4080) (width 1.0) (layer "B.Cu") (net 19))
 (segment (start 34.7980 68.3260) (end 34.7980 69.5960) (width 1.0) (layer "B.Cu") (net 13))
 (segment (start 34.7980 69.5960) (end 36.5760 71.3740) (width 1.0) (layer "B.Cu") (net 13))
 (segment (start 36.5760 71.3740) (end 36.5760 72.8980) (width 1.0) (layer "B.Cu") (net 13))
 (segment (start 26.4160 91.9480) (end 26.4160 91.4400) (width 1.0) (layer "B.Cu") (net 13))
 (segment (start 26.4160 91.4400) (end 24.6380 89.6620) (width 1.0) (layer "B.Cu") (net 13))
 (segment (start 24.6380 80.0100) (end 24.6380 79.7560) (width 1.0) (layer "B.Cu") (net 13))
 (segment (start 24.6380 79.7560) (end 27.1780 77.2160) (width 1.0) (layer "B.Cu") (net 13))
 (segment (start 27.1780 77.2160) (end 29.9720 77.2160) (width 1.0) (layer "B.Cu") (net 13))
 (segment (start 29.9720 72.1360) (end 31.2420 70.8660) (width 1.0) (layer "B.Cu") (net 13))
 (segment (start 36.5760 59.1820) (end 35.3060 59.1820) (width 1.0) (layer "B.Cu") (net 1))
 (segment (start 32.7660 59.1820) (end 34.0360 59.1820) (width 1.0) (layer "B.Cu") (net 1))
 (segment (start 26.9240 68.3260) (end 26.9240 71.1200) (width 1.0) (layer "B.Cu") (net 1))
 (segment (start 12.4460 22.8600) (end 17.5260 22.8600) (width 1.0) (layer "B.Cu") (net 1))
 (segment (start 25.6540 23.1140) (end 30.4800 23.1140) (width 1.0) (layer "B.Cu") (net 1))
 (segment (start 30.4800 47.4980) (end 25.6540 47.4980) (width 1.0) (layer "B.Cu") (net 1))
 (segment (start 14.4780 60.7060) (end 14.4780 61.2140) (width 1.0) (layer "B.Cu") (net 7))
 (segment (start 14.4780 61.2140) (end 16.2560 62.9920) (width 1.0) (layer "B.Cu") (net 7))
 (segment (start 31.2420 62.9920) (end 31.7500 62.4840) (width 1.0) (layer "B.Cu") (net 7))
 (segment (start 31.7500 62.4840) (end 38.3540 62.4840) (width 1.0) (layer "B.Cu") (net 7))
 (segment (start 38.3540 62.4840) (end 39.3700 61.4680) (width 1.0) (layer "B.Cu") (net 7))
 (segment (start 39.3700 61.4680) (end 39.3700 57.6580) (width 1.0) (layer "B.Cu") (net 7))
 (segment (start 39.3700 57.6580) (end 37.0840 55.3720) (width 1.0) (layer "B.Cu") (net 7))
 (segment (start 37.0840 55.3720) (end 29.9720 55.3720) (width 1.0) (layer "B.Cu") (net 7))
 (segment (start 29.9720 55.3720) (end 27.6860 53.0860) (width 1.0) (layer "B.Cu") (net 7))
 (segment (start 27.6860 38.8620) (end 25.6540 40.8940) (width 1.0) (layer "B.Cu") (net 7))
 (segment (start 14.7320 82.0420) (end 13.2080 82.0420) (width 1.0) (layer "B.Cu") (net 18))
 (segment (start 13.2080 89.1540) (end 10.4140 91.9480) (width 1.0) (layer "B.Cu") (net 18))
 (segment (start 10.4140 91.9480) (end 6.3500 91.9480) (width 1.0) (layer "B.Cu") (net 18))
 (segment (start 6.3500 86.8680) (end 4.0640 86.8680) (width 1.0) (layer "B.Cu") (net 18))
 (segment (start 22.0980 58.6740) (end 22.0980 57.9120) (width 1.0) (layer "B.Cu") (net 10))
 (segment (start 22.0980 57.9120) (end 24.3840 55.6260) (width 1.0) (layer "B.Cu") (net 10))
 (segment (start 24.3840 55.6260) (end 25.4000 55.6260) (width 1.0) (layer "B.Cu") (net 10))
 (segment (start 40.8940 55.6260) (end 38.1000 52.8320) (width 1.0) (layer "B.Cu") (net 10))
 (segment (start 4.3180 58.6740) (end 4.3180 53.5940) (width 1.0) (layer "B.Cu") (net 8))
 (segment (start 4.3180 53.5940) (end 4.8260 53.0860) (width 1.0) (layer "B.Cu") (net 8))
 (segment (start 19.0500 60.7060) (end 19.0500 61.7220) (width 1.0) (layer "B.Cu") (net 9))
 (segment (start 16.2560 77.9780) (end 18.7960 77.9780) (width 1.0) (layer "B.Cu") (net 16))
 (segment (start 9.6520 73.6600) (end 13.4620 73.6600) (width 1.0) (layer "B.Cu") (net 16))
 (segment (start 13.4620 73.6600) (end 14.7320 74.9300) (width 1.0) (layer "B.Cu") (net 16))
 (segment (start 14.7320 74.9300) (end 14.7320 77.9780) (width 1.0) (layer "B.Cu") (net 16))
 (segment (start 8.1280 76.9620) (end 8.1280 79.7560) (width 1.0) (layer "B.Cu") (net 15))
 (segment (start 6.8580 74.9300) (end 6.8580 75.9460) (width 1.0) (layer "B.Cu") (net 15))
 (segment (start 6.8580 75.9460) (end 7.3660 76.4540) (width 1.0) (layer "B.Cu") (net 15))
 (gr_rect (start 0 0) (end 43.0 96.0) (stroke (width 0.1) (type solid)) (fill none) (layer "Edge.Cuts"))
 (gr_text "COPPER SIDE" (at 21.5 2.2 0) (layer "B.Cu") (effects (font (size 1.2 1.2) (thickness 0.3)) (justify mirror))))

